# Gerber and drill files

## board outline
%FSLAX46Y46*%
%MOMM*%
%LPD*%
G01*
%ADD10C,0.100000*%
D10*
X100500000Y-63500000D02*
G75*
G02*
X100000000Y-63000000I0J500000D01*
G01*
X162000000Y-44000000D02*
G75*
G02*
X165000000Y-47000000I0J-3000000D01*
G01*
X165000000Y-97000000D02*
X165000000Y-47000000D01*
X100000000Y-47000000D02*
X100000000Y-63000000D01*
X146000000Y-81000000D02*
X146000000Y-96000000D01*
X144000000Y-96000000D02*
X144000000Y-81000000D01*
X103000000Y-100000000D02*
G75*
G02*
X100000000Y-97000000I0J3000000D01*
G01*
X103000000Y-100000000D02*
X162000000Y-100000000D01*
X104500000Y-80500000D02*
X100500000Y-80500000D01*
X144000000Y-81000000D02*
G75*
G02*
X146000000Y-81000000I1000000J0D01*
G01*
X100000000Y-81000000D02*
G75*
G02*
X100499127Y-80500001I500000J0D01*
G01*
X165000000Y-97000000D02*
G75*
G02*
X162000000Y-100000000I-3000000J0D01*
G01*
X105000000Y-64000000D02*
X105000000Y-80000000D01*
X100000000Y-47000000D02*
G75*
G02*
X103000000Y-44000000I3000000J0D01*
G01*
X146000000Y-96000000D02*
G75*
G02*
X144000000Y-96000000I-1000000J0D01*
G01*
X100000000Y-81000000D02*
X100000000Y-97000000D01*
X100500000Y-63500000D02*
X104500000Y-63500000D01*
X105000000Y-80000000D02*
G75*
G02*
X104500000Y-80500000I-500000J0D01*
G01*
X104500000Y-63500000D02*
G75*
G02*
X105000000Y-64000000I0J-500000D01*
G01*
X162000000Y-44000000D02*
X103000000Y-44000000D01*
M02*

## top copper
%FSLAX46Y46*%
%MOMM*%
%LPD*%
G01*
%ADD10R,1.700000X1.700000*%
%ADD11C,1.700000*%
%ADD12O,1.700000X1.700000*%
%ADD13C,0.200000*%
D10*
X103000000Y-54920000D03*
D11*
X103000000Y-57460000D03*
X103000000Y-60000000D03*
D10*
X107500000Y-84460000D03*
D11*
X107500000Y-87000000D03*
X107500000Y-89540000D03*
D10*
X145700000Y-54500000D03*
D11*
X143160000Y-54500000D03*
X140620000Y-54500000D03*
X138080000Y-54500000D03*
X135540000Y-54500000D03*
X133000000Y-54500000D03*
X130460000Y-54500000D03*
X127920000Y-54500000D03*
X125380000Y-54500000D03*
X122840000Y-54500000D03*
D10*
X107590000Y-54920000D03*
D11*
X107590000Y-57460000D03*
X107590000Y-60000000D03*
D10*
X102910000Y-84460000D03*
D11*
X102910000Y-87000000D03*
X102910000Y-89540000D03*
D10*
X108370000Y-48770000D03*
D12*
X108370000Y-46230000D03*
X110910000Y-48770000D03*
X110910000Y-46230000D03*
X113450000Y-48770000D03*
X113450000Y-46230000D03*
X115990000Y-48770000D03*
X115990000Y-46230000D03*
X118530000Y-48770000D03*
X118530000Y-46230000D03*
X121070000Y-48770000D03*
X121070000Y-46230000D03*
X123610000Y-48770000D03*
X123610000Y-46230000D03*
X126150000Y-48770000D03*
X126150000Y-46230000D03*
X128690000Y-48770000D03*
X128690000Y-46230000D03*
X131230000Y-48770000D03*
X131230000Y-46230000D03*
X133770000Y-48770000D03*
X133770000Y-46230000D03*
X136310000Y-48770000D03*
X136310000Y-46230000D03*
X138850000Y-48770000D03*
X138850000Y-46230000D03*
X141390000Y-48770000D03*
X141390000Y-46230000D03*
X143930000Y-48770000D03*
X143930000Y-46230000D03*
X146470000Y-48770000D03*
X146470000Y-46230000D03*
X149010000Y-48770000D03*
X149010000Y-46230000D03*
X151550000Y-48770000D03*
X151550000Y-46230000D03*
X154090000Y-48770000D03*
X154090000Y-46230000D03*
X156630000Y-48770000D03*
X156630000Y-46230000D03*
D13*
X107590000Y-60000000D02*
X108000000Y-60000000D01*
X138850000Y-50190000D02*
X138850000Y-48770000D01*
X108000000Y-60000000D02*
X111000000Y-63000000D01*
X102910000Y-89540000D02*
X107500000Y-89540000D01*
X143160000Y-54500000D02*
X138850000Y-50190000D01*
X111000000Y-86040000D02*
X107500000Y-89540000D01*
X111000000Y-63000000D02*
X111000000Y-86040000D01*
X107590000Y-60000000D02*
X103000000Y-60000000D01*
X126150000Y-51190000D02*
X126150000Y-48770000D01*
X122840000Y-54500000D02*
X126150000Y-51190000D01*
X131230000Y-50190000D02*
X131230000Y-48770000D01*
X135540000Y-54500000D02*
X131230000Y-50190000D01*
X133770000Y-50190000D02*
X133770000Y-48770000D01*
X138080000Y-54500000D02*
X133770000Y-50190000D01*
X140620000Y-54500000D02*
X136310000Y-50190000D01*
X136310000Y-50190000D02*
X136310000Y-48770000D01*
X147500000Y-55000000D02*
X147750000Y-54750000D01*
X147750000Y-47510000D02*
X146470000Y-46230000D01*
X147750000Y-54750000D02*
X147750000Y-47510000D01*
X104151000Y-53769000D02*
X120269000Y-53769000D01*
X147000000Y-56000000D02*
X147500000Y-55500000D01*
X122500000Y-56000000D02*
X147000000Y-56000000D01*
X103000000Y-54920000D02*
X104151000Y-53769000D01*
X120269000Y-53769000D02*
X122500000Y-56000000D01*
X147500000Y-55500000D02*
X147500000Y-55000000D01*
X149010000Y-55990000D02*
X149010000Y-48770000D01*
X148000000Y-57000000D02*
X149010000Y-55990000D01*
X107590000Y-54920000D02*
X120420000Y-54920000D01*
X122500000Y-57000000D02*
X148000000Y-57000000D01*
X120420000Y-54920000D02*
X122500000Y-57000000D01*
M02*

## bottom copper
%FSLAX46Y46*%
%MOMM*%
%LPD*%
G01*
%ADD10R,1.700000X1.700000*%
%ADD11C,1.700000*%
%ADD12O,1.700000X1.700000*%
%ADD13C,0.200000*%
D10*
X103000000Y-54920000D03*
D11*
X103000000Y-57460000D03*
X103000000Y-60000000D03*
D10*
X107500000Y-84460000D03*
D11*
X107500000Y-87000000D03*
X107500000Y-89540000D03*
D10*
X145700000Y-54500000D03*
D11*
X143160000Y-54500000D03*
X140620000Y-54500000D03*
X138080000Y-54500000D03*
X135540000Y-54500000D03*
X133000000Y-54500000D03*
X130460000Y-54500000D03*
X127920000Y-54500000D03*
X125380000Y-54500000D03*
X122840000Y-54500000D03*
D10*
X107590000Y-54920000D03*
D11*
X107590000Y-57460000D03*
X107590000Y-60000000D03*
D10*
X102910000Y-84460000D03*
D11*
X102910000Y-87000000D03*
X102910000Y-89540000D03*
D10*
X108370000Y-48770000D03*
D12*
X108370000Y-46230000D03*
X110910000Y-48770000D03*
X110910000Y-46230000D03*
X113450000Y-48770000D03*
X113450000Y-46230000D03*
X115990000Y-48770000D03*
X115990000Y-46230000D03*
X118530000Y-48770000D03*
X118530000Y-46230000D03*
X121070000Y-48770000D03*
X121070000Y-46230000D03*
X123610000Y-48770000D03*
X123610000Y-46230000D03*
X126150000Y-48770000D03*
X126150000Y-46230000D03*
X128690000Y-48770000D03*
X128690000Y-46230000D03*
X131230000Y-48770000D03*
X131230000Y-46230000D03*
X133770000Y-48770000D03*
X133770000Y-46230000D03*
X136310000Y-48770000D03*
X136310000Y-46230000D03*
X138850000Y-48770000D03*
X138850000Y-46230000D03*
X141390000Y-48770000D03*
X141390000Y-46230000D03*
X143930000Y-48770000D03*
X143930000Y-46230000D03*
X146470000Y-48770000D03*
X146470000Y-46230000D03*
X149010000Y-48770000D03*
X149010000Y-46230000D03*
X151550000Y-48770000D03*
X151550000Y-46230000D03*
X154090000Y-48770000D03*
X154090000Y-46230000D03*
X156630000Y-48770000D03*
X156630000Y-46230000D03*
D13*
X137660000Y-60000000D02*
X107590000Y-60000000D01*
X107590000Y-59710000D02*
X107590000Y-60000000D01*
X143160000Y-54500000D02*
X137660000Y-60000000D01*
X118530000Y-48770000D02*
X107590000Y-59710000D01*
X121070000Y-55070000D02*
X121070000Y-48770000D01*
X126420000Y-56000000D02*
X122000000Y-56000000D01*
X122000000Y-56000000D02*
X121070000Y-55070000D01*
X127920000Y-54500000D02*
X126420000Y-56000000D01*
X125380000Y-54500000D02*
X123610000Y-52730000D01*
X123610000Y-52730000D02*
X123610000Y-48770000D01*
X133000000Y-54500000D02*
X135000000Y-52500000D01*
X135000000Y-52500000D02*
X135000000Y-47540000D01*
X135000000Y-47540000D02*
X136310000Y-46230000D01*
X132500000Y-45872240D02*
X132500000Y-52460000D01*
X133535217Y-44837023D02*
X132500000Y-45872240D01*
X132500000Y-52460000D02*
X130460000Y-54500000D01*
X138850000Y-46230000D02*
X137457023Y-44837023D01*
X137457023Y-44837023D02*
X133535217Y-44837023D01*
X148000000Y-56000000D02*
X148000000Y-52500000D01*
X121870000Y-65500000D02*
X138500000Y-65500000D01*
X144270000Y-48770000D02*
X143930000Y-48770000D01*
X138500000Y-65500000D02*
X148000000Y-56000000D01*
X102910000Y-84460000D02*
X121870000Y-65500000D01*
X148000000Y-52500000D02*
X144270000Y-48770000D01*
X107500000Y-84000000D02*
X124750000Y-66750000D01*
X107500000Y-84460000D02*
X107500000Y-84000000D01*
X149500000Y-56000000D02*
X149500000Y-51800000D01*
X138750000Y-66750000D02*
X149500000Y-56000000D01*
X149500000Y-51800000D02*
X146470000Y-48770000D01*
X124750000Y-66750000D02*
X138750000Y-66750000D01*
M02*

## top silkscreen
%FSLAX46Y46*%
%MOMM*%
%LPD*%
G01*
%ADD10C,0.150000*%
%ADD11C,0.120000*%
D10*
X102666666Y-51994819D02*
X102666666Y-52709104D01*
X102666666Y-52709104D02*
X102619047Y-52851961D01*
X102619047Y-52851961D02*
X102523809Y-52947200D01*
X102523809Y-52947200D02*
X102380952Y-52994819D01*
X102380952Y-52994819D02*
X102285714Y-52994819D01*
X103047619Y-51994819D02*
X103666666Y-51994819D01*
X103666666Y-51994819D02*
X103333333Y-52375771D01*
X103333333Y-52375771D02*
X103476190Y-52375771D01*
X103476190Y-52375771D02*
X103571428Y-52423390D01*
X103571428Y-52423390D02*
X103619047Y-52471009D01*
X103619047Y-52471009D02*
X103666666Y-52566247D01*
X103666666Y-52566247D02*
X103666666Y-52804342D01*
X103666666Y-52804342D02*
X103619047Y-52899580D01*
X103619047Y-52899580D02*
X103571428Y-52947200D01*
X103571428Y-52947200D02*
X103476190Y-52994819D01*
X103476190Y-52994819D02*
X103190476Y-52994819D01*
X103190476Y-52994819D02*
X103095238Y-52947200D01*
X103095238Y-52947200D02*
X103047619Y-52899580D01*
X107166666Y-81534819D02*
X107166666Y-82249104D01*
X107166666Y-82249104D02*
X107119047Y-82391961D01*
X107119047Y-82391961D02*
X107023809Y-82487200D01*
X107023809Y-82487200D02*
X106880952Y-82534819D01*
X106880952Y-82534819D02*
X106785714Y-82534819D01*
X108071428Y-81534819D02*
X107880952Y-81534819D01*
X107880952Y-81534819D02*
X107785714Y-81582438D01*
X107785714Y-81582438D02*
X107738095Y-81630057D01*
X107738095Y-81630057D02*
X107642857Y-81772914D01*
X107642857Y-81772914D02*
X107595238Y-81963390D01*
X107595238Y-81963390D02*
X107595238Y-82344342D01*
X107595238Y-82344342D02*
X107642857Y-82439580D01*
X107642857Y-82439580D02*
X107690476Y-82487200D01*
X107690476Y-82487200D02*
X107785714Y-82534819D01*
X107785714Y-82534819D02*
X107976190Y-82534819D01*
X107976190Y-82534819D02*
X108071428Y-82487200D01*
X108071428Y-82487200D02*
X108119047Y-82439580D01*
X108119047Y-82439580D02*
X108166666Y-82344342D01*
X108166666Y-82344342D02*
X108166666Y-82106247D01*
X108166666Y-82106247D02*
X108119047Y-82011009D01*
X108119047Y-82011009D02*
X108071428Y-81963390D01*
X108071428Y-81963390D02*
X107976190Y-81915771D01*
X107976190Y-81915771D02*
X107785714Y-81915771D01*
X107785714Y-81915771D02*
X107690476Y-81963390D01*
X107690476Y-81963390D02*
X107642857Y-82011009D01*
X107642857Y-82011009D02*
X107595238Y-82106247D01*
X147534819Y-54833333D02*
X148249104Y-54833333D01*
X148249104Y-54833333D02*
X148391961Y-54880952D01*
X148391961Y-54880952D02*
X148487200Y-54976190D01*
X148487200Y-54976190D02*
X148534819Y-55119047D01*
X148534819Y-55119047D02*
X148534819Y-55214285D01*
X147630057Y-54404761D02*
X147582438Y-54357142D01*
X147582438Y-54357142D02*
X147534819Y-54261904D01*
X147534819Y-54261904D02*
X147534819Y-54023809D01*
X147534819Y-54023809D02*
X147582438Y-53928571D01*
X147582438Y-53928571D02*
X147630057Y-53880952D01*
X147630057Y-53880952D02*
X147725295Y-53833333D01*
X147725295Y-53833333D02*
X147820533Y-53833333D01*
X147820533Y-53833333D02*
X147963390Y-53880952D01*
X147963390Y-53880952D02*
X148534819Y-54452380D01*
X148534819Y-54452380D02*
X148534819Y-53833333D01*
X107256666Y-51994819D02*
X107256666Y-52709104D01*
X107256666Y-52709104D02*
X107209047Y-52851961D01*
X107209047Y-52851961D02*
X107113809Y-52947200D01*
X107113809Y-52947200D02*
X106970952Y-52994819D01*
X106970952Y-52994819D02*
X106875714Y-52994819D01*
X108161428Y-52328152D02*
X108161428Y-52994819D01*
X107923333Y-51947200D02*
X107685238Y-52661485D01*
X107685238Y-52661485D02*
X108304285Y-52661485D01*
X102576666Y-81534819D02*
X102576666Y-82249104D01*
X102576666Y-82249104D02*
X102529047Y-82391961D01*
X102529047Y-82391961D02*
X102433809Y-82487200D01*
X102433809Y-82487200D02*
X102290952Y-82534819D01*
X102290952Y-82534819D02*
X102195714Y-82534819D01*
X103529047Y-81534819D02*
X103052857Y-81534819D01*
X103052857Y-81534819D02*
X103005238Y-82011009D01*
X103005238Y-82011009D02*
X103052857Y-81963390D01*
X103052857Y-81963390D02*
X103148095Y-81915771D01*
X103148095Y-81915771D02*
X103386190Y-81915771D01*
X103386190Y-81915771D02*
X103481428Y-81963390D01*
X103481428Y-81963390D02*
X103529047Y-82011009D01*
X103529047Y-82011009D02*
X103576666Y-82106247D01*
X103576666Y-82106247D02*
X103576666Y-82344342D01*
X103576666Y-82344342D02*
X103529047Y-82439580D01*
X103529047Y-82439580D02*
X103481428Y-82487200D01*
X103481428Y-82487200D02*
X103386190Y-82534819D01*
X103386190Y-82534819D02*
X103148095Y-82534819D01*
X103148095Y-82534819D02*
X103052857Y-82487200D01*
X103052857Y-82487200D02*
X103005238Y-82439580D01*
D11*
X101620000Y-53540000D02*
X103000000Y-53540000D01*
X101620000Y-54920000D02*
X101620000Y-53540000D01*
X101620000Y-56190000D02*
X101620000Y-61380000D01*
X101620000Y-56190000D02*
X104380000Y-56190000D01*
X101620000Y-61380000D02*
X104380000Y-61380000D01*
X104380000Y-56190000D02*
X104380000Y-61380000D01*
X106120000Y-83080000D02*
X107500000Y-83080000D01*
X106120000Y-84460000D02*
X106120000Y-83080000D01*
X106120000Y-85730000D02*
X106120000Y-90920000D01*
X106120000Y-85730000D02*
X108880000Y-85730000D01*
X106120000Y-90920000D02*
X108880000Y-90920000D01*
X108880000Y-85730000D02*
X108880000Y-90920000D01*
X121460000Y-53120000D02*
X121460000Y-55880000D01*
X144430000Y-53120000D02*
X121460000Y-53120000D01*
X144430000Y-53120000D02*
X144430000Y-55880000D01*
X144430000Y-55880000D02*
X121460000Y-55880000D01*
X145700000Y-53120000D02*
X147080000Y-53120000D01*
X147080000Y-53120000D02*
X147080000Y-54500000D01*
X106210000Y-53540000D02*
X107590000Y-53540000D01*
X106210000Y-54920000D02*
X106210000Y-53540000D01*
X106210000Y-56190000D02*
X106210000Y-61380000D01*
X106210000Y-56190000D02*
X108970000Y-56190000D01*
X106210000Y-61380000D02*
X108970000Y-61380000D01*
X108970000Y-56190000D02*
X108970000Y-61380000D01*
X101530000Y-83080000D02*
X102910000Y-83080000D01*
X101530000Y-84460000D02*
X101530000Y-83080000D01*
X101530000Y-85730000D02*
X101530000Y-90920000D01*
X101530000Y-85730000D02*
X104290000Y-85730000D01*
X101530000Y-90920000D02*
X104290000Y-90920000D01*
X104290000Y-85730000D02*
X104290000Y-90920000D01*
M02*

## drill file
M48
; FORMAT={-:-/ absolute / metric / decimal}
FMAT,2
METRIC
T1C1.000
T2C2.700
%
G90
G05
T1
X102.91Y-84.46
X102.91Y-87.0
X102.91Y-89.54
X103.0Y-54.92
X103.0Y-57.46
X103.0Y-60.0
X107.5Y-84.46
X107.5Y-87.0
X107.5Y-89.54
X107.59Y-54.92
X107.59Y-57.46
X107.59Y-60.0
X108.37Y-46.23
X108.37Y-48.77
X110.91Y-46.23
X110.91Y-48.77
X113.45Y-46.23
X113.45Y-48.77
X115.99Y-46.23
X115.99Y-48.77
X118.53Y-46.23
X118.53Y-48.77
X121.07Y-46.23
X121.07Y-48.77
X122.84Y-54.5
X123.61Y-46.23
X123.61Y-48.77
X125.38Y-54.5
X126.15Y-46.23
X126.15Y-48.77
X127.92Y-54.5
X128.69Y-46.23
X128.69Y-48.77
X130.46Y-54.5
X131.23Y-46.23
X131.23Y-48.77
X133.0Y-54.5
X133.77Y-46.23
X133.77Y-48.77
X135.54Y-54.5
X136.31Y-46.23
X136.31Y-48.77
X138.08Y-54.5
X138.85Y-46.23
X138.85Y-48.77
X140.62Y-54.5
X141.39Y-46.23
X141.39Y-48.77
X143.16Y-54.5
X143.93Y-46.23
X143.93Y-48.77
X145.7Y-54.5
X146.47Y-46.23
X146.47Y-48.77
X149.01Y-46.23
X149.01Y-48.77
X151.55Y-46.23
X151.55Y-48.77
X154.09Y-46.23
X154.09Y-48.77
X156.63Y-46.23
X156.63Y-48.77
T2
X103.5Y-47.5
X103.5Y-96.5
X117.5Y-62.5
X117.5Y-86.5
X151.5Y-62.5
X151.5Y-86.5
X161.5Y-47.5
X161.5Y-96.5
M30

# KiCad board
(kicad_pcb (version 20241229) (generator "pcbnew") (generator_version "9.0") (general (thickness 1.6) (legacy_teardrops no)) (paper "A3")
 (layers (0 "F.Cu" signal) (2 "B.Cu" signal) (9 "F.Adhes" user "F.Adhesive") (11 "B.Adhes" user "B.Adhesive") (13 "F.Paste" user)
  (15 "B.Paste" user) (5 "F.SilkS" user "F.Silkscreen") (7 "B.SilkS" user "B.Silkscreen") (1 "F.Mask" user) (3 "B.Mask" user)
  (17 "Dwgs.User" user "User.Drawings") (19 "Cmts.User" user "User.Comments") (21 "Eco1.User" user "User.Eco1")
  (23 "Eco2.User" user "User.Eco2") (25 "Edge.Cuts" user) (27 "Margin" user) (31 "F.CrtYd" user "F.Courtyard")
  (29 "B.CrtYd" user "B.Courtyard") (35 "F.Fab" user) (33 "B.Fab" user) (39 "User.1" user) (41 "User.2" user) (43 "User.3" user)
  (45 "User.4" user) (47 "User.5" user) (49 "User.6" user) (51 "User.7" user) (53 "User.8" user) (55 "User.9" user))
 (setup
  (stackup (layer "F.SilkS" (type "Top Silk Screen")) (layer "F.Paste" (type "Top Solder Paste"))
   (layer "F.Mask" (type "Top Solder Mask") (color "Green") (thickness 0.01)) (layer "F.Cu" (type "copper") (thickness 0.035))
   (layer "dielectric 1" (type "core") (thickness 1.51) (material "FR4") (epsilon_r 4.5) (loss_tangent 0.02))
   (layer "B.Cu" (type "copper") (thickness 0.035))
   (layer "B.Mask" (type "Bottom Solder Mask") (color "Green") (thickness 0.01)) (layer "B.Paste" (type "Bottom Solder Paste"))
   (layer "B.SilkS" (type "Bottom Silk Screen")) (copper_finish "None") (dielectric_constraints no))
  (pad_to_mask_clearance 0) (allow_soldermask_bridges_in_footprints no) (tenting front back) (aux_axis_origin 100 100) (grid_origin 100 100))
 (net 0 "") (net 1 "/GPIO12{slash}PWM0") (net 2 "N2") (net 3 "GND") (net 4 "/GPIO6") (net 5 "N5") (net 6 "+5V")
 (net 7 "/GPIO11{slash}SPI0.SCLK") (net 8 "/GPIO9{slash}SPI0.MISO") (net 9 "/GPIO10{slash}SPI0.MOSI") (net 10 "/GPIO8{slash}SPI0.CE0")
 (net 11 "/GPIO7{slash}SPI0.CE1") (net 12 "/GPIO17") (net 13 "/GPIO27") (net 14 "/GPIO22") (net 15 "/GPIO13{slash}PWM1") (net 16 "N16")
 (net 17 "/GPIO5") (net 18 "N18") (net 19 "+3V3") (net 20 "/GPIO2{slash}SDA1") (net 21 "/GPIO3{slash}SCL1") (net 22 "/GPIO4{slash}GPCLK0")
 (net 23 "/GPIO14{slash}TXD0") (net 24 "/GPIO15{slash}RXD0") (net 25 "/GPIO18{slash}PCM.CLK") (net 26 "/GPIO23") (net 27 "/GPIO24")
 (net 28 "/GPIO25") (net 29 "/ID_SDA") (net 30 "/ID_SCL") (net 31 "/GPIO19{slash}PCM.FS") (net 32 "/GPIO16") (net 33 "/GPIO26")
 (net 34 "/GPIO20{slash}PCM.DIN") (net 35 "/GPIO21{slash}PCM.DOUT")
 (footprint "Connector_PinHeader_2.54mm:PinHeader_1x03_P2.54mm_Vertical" (layer "F.Cu") (at 103 54.92)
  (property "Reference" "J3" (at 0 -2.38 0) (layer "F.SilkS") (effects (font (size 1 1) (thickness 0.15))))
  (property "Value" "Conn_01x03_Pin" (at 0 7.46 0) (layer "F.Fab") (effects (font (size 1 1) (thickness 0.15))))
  (fp_line (start -1.38 -1.38) (end 0 -1.38) (stroke (width 0.12) (type solid)) (layer "F.SilkS"))
  (fp_line (start -1.38 0) (end -1.38 -1.38) (stroke (width 0.12) (type solid)) (layer "F.SilkS"))
  (fp_line (start -1.38 1.27) (end -1.38 6.46) (stroke (width 0.12) (type solid)) (layer "F.SilkS"))
  (fp_line (start -1.38 1.27) (end 1.38 1.27) (stroke (width 0.12) (type solid)) (layer "F.SilkS"))
  (fp_line (start -1.38 6.46) (end 1.38 6.46) (stroke (width 0.12) (type solid)) (layer "F.SilkS"))
  (fp_line (start 1.38 1.27) (end 1.38 6.46) (stroke (width 0.12) (type solid)) (layer "F.SilkS"))
  (pad "1" thru_hole rect (at 0 0) (size 1.7 1.7) (drill 1) (layers "*.Cu" "*.Mask") (remove_unused_layers no) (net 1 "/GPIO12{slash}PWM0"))
  (pad "2" thru_hole circle (at 0 2.54) (size 1.7 1.7) (drill 1) (layers "*.Cu" "*.Mask") (remove_unused_layers no) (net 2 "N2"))
  (pad "3" thru_hole circle (at 0 5.08) (size 1.7 1.7) (drill 1) (layers "*.Cu" "*.Mask") (remove_unused_layers no) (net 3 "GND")))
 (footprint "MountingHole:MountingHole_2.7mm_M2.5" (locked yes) (layer "F.Cu") (at 161.5 47.5)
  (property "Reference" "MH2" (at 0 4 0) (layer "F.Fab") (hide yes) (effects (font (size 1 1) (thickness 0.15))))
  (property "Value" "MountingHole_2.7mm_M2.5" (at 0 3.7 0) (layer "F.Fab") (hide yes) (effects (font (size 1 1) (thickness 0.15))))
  (pad "" np_thru_hole circle (at 0 0) (size 2.7 2.7) (drill 2.7) (layers "*.Cu" "*.Mask")))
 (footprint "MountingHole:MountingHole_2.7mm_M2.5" (layer "F.Cu") (at 117.5 86.5)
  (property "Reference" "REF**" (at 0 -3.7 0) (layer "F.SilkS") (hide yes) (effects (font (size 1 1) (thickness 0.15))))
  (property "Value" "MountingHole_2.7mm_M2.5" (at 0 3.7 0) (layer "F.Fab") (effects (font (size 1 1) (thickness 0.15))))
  (pad "" np_thru_hole circle (at 0 0) (size 2.7 2.7) (drill 2.7) (layers "*.Cu" "*.Mask")))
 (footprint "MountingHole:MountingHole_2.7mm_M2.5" (layer "F.Cu") (at 151.5 86.5)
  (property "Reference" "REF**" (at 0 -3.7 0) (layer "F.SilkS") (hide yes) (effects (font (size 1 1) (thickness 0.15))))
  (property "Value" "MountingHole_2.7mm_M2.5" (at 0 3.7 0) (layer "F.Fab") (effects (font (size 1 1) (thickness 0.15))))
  (pad "" np_thru_hole circle (at 0 0) (size 2.7 2.7) (drill 2.7) (layers "*.Cu" "*.Mask")))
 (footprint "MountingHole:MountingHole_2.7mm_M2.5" (layer "F.Cu") (at 151.5 62.5)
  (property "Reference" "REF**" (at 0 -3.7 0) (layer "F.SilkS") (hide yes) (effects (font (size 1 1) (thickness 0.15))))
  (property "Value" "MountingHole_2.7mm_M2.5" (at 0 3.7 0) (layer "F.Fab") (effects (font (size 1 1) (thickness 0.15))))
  (pad "" np_thru_hole circle (at 0 0) (size 2.7 2.7) (drill 2.7) (layers "*.Cu" "*.Mask")))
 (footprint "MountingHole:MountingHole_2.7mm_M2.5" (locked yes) (layer "F.Cu") (at 103.5 96.5)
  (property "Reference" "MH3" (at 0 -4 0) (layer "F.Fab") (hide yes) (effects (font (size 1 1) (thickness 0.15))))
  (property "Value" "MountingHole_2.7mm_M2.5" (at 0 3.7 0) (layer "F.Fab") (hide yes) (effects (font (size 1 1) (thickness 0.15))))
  (pad "" np_thru_hole circle (at 0 0) (size 2.7 2.7) (drill 2.7) (layers "*.Cu" "*.Mask")))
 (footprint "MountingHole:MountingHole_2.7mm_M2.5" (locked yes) (layer "F.Cu") (at 103.5 47.5)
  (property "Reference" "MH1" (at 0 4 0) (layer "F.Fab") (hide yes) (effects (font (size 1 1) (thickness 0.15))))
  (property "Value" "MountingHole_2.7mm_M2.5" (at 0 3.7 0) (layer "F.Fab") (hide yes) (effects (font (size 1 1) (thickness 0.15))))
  (pad "" np_thru_hole circle (at 0 0) (size 2.7 2.7) (drill 2.7) (layers "*.Cu" "*.Mask")))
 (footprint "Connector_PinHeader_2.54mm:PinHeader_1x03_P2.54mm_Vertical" (layer "F.Cu") (at 107.5 84.46)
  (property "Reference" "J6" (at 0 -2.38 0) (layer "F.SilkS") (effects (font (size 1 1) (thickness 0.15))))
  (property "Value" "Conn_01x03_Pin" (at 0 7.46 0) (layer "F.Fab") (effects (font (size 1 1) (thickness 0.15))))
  (fp_line (start -1.38 -1.38) (end 0 -1.38) (stroke (width 0.12) (type solid)) (layer "F.SilkS"))
  (fp_line (start -1.38 0) (end -1.38 -1.38) (stroke (width 0.12) (type solid)) (layer "F.SilkS"))
  (fp_line (start -1.38 1.27) (end -1.38 6.46) (stroke (width 0.12) (type solid)) (layer "F.SilkS"))
  (fp_line (start -1.38 1.27) (end 1.38 1.27) (stroke (width 0.12) (type solid)) (layer "F.SilkS"))
  (fp_line (start -1.38 6.46) (end 1.38 6.46) (stroke (width 0.12) (type solid)) (layer "F.SilkS"))
  (fp_line (start 1.38 1.27) (end 1.38 6.46) (stroke (width 0.12) (type solid)) (layer "F.SilkS"))
  (pad "1" thru_hole rect (at 0 0) (size 1.7 1.7) (drill 1) (layers "*.Cu" "*.Mask") (remove_unused_layers no) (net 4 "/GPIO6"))
  (pad "2" thru_hole circle (at 0 2.54) (size 1.7 1.7) (drill 1) (layers "*.Cu" "*.Mask") (remove_unused_layers no) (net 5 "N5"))
  (pad "3" thru_hole circle (at 0 5.08) (size 1.7 1.7) (drill 1) (layers "*.Cu" "*.Mask") (remove_unused_layers no) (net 3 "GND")))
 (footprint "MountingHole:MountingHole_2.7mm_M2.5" (layer "F.Cu") (at 117.5 62.5)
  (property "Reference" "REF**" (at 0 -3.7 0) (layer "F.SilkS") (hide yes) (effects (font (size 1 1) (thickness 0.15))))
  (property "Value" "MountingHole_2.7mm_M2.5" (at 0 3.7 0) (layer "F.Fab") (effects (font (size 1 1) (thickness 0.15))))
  (pad "" np_thru_hole circle (at 0 0) (size 2.7 2.7) (drill 2.7) (layers "*.Cu" "*.Mask")))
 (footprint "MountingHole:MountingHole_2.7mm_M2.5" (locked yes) (layer "F.Cu") (at 161.5 96.5)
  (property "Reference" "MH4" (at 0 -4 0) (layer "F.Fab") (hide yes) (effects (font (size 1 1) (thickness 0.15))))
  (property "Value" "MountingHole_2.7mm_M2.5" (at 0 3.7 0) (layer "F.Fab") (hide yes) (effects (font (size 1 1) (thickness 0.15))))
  (pad "" np_thru_hole circle (at 0 0) (size 2.7 2.7) (drill 2.7) (layers "*.Cu" "*.Mask")))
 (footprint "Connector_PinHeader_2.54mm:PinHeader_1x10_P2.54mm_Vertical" (layer "F.Cu") (at 145.7 54.5 -90)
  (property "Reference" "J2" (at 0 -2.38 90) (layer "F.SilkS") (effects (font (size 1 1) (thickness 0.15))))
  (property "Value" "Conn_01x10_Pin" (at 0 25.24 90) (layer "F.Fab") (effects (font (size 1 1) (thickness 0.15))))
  (fp_line (start -1.38 24.24) (end 1.38 24.24) (stroke (width 0.12) (type solid)) (layer "F.SilkS"))
  (fp_line (start -1.38 1.27) (end -1.38 24.24) (stroke (width 0.12) (type solid)) (layer "F.SilkS"))
  (fp_line (start -1.38 1.27) (end 1.38 1.27) (stroke (width 0.12) (type solid)) (layer "F.SilkS"))
  (fp_line (start 1.38 1.27) (end 1.38 24.24) (stroke (width 0.12) (type solid)) (layer "F.SilkS"))
  (fp_line (start -1.38 0) (end -1.38 -1.38) (stroke (width 0.12) (type solid)) (layer "F.SilkS"))
  (fp_line (start -1.38 -1.38) (end 0 -1.38) (stroke (width 0.12) (type solid)) (layer "F.SilkS"))
  (pad "1" thru_hole rect (at 0 0 270) (size 1.7 1.7) (drill 1) (layers "*.Cu" "*.Mask") (remove_unused_layers no) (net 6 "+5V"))
  (pad "2" thru_hole circle (at 0 2.54 270) (size 1.7 1.7) (drill 1) (layers "*.Cu" "*.Mask") (remove_unused_layers no) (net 3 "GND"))
  (pad "3" thru_hole circle (at 0 5.08 270) (size 1.7 1.7) (drill 1) (layers "*.Cu" "*.Mask") (remove_unused_layers no)
   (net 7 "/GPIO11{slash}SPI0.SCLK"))
  (pad "4" thru_hole circle (at 0 7.62 270) (size 1.7 1.7) (drill 1) (layers "*.Cu" "*.Mask") (remove_unused_layers no)
   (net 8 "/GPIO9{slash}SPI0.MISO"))
  (pad "5" thru_hole circle (at 0 10.16 270) (size 1.7 1.7) (drill 1) (layers "*.Cu" "*.Mask") (remove_unused_layers no)
   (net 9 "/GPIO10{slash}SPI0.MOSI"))
  (pad "6" thru_hole circle (at 0 12.7 270) (size 1.7 1.7) (drill 1) (layers "*.Cu" "*.Mask") (remove_unused_layers no)
   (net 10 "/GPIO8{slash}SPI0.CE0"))
  (pad "7" thru_hole circle (at 0 15.24 270) (size 1.7 1.7) (drill 1) (layers "*.Cu" "*.Mask") (remove_unused_layers no)
   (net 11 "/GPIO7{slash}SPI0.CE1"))
  (pad "8" thru_hole circle (at 0 17.78 270) (size 1.7 1.7) (drill 1) (layers "*.Cu" "*.Mask") (remove_unused_layers no) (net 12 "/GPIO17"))
  (pad "9" thru_hole circle (at 0 20.32 270) (size 1.7 1.7) (drill 1) (layers "*.Cu" "*.Mask") (remove_unused_layers no) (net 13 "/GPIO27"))
  (pad "10" thru_hole circle (at 0 22.86 270) (size 1.7 1.7) (drill 1) (layers "*.Cu" "*.Mask") (remove_unused_layers no) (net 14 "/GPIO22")))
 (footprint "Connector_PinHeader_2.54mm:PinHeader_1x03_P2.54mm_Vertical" (layer "F.Cu") (at 107.59 54.92)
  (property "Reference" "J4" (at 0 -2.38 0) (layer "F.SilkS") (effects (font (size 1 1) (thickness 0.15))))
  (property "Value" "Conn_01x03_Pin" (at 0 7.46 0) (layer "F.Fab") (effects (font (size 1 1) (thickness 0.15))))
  (fp_line (start -1.38 -1.38) (end 0 -1.38) (stroke (width 0.12) (type solid)) (layer "F.SilkS"))
  (fp_line (start -1.38 0) (end -1.38 -1.38) (stroke (width 0.12) (type solid)) (layer "F.SilkS"))
  (fp_line (start -1.38 1.27) (end -1.38 6.46) (stroke (width 0.12) (type solid)) (layer "F.SilkS"))
  (fp_line (start -1.38 1.27) (end 1.38 1.27) (stroke (width 0.12) (type solid)) (layer "F.SilkS"))
  (fp_line (start -1.38 6.46) (end 1.38 6.46) (stroke (width 0.12) (type solid)) (layer "F.SilkS"))
  (fp_line (start 1.38 1.27) (end 1.38 6.46) (stroke (width 0.12) (type solid)) (layer "F.SilkS"))
  (pad "1" thru_hole rect (at 0 0) (size 1.7 1.7) (drill 1) (layers "*.Cu" "*.Mask") (remove_unused_layers no) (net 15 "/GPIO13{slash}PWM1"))
  (pad "2" thru_hole circle (at 0 2.54) (size 1.7 1.7) (drill 1) (layers "*.Cu" "*.Mask") (remove_unused_layers no) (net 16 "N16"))
  (pad "3" thru_hole circle (at 0 5.08) (size 1.7 1.7) (drill 1) (layers "*.Cu" "*.Mask") (remove_unused_layers no) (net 3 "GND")))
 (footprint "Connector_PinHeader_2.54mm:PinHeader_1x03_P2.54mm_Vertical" (layer "F.Cu") (at 102.91 84.46)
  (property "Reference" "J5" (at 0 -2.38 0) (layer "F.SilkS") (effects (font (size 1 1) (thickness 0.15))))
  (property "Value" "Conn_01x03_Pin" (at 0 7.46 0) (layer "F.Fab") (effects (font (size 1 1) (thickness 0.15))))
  (fp_line (start -1.38 -1.38) (end 0 -1.38) (stroke (width 0.12) (type solid)) (layer "F.SilkS"))
  (fp_line (start -1.38 0) (end -1.38 -1.38) (stroke (width 0.12) (type solid)) (layer "F.SilkS"))
  (fp_line (start -1.38 1.27) (end -1.38 6.46) (stroke (width 0.12) (type solid)) (layer "F.SilkS"))
  (fp_line (start -1.38 1.27) (end 1.38 1.27) (stroke (width 0.12) (type solid)) (layer "F.SilkS"))
  (fp_line (start -1.38 6.46) (end 1.38 6.46) (stroke (width 0.12) (type solid)) (layer "F.SilkS"))
  (fp_line (start 1.38 1.27) (end 1.38 6.46) (stroke (width 0.12) (type solid)) (layer "F.SilkS"))
  (pad "1" thru_hole rect (at 0 0) (size 1.7 1.7) (drill 1) (layers "*.Cu" "*.Mask") (remove_unused_layers no) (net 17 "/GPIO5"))
  (pad "2" thru_hole circle (at 0 2.54) (size 1.7 1.7) (drill 1) (layers "*.Cu" "*.Mask") (remove_unused_layers no) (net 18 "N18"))
  (pad "3" thru_hole circle (at 0 5.08) (size 1.7 1.7) (drill 1) (layers "*.Cu" "*.Mask") (remove_unused_layers no) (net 3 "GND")))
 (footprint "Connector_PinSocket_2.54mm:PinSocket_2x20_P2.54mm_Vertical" (layer "B.Cu") (at 108.37 48.77 -90)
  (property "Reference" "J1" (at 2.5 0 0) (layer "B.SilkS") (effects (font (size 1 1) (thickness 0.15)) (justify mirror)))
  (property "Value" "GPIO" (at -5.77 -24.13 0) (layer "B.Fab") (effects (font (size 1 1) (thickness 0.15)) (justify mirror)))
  (pad "1" thru_hole rect (at 0 0 270) (size 1.7 1.7) (drill 1) (layers "*.Cu" "*.Mask") (remove_unused_layers no) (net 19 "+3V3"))
  (pad "2" thru_hole oval (at -2.54 0 270) (size 1.7 1.7) (drill 1) (layers "*.Cu" "*.Mask") (remove_unused_layers no) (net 6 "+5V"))
  (pad "3" thru_hole oval (at 0 -2.54 270) (size 1.7 1.7) (drill 1) (layers "*.Cu" "*.Mask") (remove_unused_layers no)
   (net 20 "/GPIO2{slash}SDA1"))
  (pad "4" thru_hole oval (at -2.54 -2.54 270) (size 1.7 1.7) (drill 1) (layers "*.Cu" "*.Mask") (remove_unused_layers no) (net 6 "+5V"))
  (pad "5" thru_hole oval (at 0 -5.08 270) (size 1.7 1.7) (drill 1) (layers "*.Cu" "*.Mask") (remove_unused_layers no)
   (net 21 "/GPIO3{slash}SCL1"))
  (pad "6" thru_hole oval (at -2.54 -5.08 270) (size 1.7 1.7) (drill 1) (layers "*.Cu" "*.Mask") (remove_unused_layers no) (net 3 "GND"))
  (pad "7" thru_hole oval (at 0 -7.62 270) (size 1.7 1.7) (drill 1) (layers "*.Cu" "*.Mask") (remove_unused_layers no)
   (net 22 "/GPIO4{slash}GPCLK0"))
  (pad "8" thru_hole oval (at -2.54 -7.62 270) (size 1.7 1.7) (drill 1) (layers "*.Cu" "*.Mask") (remove_unused_layers no)
   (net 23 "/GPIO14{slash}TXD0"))
  (pad "9" thru_hole oval (at 0 -10.16 270) (size 1.7 1.7) (drill 1) (layers "*.Cu" "*.Mask") (remove_unused_layers no) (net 3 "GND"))
  (pad "10" thru_hole oval (at -2.54 -10.16 270) (size 1.7 1.7) (drill 1) (layers "*.Cu" "*.Mask") (remove_unused_layers no)
   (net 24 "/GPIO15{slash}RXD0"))
  (pad "11" thru_hole oval (at 0 -12.7 270) (size 1.7 1.7) (drill 1) (layers "*.Cu" "*.Mask") (remove_unused_layers no) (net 12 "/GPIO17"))
  (pad "12" thru_hole oval (at -2.54 -12.7 270) (size 1.7 1.7) (drill 1) (layers "*.Cu" "*.Mask") (remove_unused_layers no)
   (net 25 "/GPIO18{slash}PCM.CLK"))
  (pad "13" thru_hole oval (at 0 -15.24 270) (size 1.7 1.7) (drill 1) (layers "*.Cu" "*.Mask") (remove_unused_layers no) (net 13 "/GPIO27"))
  (pad "14" thru_hole oval (at -2.54 -15.24 270) (size 1.7 1.7) (drill 1) (layers "*.Cu" "*.Mask") (remove_unused_layers no) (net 3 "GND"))
  (pad "15" thru_hole oval (at 0 -17.78 270) (size 1.7 1.7) (drill 1) (layers "*.Cu" "*.Mask") (remove_unused_layers no) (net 14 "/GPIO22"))
  (pad "16" thru_hole oval (at -2.54 -17.78 270) (size 1.7 1.7) (drill 1) (layers "*.Cu" "*.Mask") (remove_unused_layers no)
   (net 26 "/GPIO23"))
  (pad "17" thru_hole oval (at 0 -20.32 270) (size 1.7 1.7) (drill 1) (layers "*.Cu" "*.Mask") (remove_unused_layers no) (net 19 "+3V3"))
  (pad "18" thru_hole oval (at -2.54 -20.32 270) (size 1.7 1.7) (drill 1) (layers "*.Cu" "*.Mask") (remove_unused_layers no)
   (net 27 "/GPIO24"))
  (pad "19" thru_hole oval (at 0 -22.86 270) (size 1.7 1.7) (drill 1) (layers "*.Cu" "*.Mask") (remove_unused_layers no)
   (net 9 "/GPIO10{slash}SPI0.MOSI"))
  (pad "20" thru_hole oval (at -2.54 -22.86 270) (size 1.7 1.7) (drill 1) (layers "*.Cu" "*.Mask") (remove_unused_layers no) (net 3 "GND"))
  (pad "21" thru_hole oval (at 0 -25.4 270) (size 1.7 1.7) (drill 1) (layers "*.Cu" "*.Mask") (remove_unused_layers no)
   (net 8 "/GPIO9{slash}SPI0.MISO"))
  (pad "22" thru_hole oval (at -2.54 -25.4 270) (size 1.7 1.7) (drill 1) (layers "*.Cu" "*.Mask") (remove_unused_layers no)
   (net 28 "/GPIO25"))
  (pad "23" thru_hole oval (at 0 -27.94 270) (size 1.7 1.7) (drill 1) (layers "*.Cu" "*.Mask") (remove_unused_layers no)
   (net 7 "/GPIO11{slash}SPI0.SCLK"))
  (pad "24" thru_hole oval (at -2.54 -27.94 270) (size 1.7 1.7) (drill 1) (layers "*.Cu" "*.Mask") (remove_unused_layers no)
   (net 10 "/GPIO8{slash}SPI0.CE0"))
  (pad "25" thru_hole oval (at 0 -30.48 270) (size 1.7 1.7) (drill 1) (layers "*.Cu" "*.Mask") (remove_unused_layers no) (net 3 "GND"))
  (pad "26" thru_hole oval (at -2.54 -30.48 270) (size 1.7 1.7) (drill 1) (layers "*.Cu" "*.Mask") (remove_unused_layers no)
   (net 11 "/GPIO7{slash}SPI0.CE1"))
  (pad "27" thru_hole oval (at 0 -33.02 270) (size 1.7 1.7) (drill 1) (layers "*.Cu" "*.Mask") (remove_unused_layers no) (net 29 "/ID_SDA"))
  (pad "28" thru_hole oval (at -2.54 -33.02 270) (size 1.7 1.7) (drill 1) (layers "*.Cu" "*.Mask") (remove_unused_layers no)
   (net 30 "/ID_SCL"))
  (pad "29" thru_hole oval (at 0 -35.56 270) (size 1.7 1.7) (drill 1) (layers "*.Cu" "*.Mask") (remove_unused_layers no) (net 17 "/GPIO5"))
  (pad "30" thru_hole oval (at -2.54 -35.56 270) (size 1.7 1.7) (drill 1) (layers "*.Cu" "*.Mask") (remove_unused_layers no) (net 3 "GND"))
  (pad "31" thru_hole oval (at 0 -38.1 270) (size 1.7 1.7) (drill 1) (layers "*.Cu" "*.Mask") (remove_unused_layers no) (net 4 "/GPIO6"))
  (pad "32" thru_hole oval (at -2.54 -38.1 270) (size 1.7 1.7) (drill 1) (layers "*.Cu" "*.Mask") (remove_unused_layers no)
   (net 1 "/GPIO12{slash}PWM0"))
  (pad "33" thru_hole oval (at 0 -40.64 270) (size 1.7 1.7) (drill 1) (layers "*.Cu" "*.Mask") (remove_unused_layers no)
   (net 15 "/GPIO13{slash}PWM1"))
  (pad "34" thru_hole oval (at -2.54 -40.64 270) (size 1.7 1.7) (drill 1) (layers "*.Cu" "*.Mask") (remove_unused_layers no) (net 3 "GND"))
  (pad "35" thru_hole oval (at 0 -43.18 270) (size 1.7 1.7) (drill 1) (layers "*.Cu" "*.Mask") (remove_unused_layers no)
   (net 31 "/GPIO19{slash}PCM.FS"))
  (pad "36" thru_hole oval (at -2.54 -43.18 270) (size 1.7 1.7) (drill 1) (layers "*.Cu" "*.Mask") (remove_unused_layers no)
   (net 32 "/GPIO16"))
  (pad "37" thru_hole oval (at 0 -45.72 270) (size 1.7 1.7) (drill 1) (layers "*.Cu" "*.Mask") (remove_unused_layers no) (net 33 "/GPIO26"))
  (pad "38" thru_hole oval (at -2.54 -45.72 270) (size 1.7 1.7) (drill 1) (layers "*.Cu" "*.Mask") (remove_unused_layers no)
   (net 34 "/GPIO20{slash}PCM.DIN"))
  (pad "39" thru_hole oval (at 0 -48.26 270) (size 1.7 1.7) (drill 1) (layers "*.Cu" "*.Mask") (remove_unused_layers no) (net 3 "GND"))
  (pad "40" thru_hole oval (at -2.54 -48.26 270) (size 1.7 1.7) (drill 1) (layers "*.Cu" "*.Mask") (remove_unused_layers no)
   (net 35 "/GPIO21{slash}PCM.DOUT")))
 (gr_arc (start 100.5 63.5) (mid 100.146447 63.353553) (end 100 63) (stroke (width 0.1) (type solid)) (layer "Edge.Cuts"))
 (gr_arc (start 162 44) (mid 164.12132 44.87868) (end 165 47) (stroke (width 0.1) (type solid)) (layer "Edge.Cuts"))
 (gr_line (start 165 97) (end 165 47) (stroke (width 0.1) (type solid)) (layer "Edge.Cuts"))
 (gr_line (start 100 47) (end 100 63) (stroke (width 0.1) (type solid)) (layer "Edge.Cuts"))
 (gr_line (start 146 81) (end 146 96) (stroke (width 0.1) (type solid)) (layer "Edge.Cuts"))
 (gr_line (start 144 96) (end 144 81) (stroke (width 0.1) (type solid)) (layer "Edge.Cuts"))
 (gr_arc (start 103 100) (mid 100.87868 99.12132) (end 100 97) (stroke (width 0.1) (type solid)) (layer "Edge.Cuts"))
 (gr_line (start 103 100) (end 162 100) (stroke (width 0.1) (type solid)) (layer "Edge.Cuts"))
 (gr_line (start 104.5 80.5) (end 100.5 80.5) (stroke (width 0.1) (type solid)) (layer "Edge.Cuts"))
 (gr_arc (start 144 81) (mid 145 80) (end 146 81) (stroke (width 0.1) (type solid)) (layer "Edge.Cuts"))
 (gr_arc (start 100 81) (mid 100.146138 80.646755) (end 100.499127 80.500001) (stroke (width 0.1) (type solid)) (layer "Edge.Cuts"))
 (gr_arc (start 165 97) (mid 164.12132 99.12132) (end 162 100) (stroke (width 0.1) (type solid)) (layer "Edge.Cuts"))
 (gr_line (start 105 64) (end 105 80) (stroke (width 0.1) (type solid)) (layer "Edge.Cuts"))
 (gr_arc (start 100 47) (mid 100.87868 44.87868) (end 103 44) (stroke (width 0.1) (type solid)) (layer "Edge.Cuts"))
 (gr_arc (start 146 96) (mid 145 97) (end 144 96) (stroke (width 0.1) (type solid)) (layer "Edge.Cuts"))
 (gr_line (start 100 81) (end 100 97) (stroke (width 0.1) (type solid)) (layer "Edge.Cuts"))
 (gr_line (start 100.5 63.5) (end 104.5 63.5) (stroke (width 0.1) (type solid)) (layer "Edge.Cuts"))
 (gr_arc (start 105 80) (mid 104.853553 80.353553) (end 104.5 80.5) (stroke (width 0.1) (type solid)) (layer "Edge.Cuts"))
 (gr_arc (start 104.5 63.5) (mid 104.853553 63.646447) (end 105 64) (stroke (width 0.1) (type solid)) (layer "Edge.Cuts"))
 (gr_line (start 162 44) (end 103 44) (stroke (width 0.1) (type solid)) (layer "Edge.Cuts"))
 (segment (start 107.59 60) (end 108 60) (width 0.2) (layer "F.Cu") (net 3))
 (segment (start 138.85 50.19) (end 138.85 48.77) (width 0.2) (layer "F.Cu") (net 3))
 (segment (start 108 60) (end 111 63) (width 0.2) (layer "F.Cu") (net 3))
 (segment (start 102.91 89.54) (end 107.5 89.54) (width 0.2) (layer "F.Cu") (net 3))
 (segment (start 143.16 54.5) (end 138.85 50.19) (width 0.2) (layer "F.Cu") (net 3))
 (segment (start 111 86.04) (end 107.5 89.54) (width 0.2) (layer "F.Cu") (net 3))
 (segment (start 111 63) (end 111 86.04) (width 0.2) (layer "F.Cu") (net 3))
 (segment (start 107.59 60) (end 103 60) (width 0.2) (layer "F.Cu") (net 3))
 (segment (start 137.66 60) (end 107.59 60) (width 0.2) (layer "B.Cu") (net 3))
 (segment (start 107.59 59.71) (end 107.59 60) (width 0.2) (layer "B.Cu") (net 3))
 (segment (start 143.16 54.5) (end 137.66 60) (width 0.2) (layer "B.Cu") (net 3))
 (segment (start 118.53 48.77) (end 107.59 59.71) (width 0.2) (layer "B.Cu") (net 3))
 (segment (start 121.07 55.07) (end 121.07 48.77) (width 0.2) (layer "B.Cu") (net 12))
 (segment (start 126.42 56) (end 122 56) (width 0.2) (layer "B.Cu") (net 12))
 (segment (start 122 56) (end 121.07 55.07) (width 0.2) (layer "B.Cu") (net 12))
 (segment (start 127.92 54.5) (end 126.42 56) (width 0.2) (layer "B.Cu") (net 12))
 (segment (start 125.38 54.5) (end 123.61 52.73) (width 0.2) (layer "B.Cu") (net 13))
 (segment (start 123.61 52.73) (end 123.61 48.77) (width 0.2) (layer "B.Cu") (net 13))
 (segment (start 126.15 51.19) (end 126.15 48.77) (width 0.2) (layer "F.Cu") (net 14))
 (segment (start 122.84 54.5) (end 126.15 51.19) (width 0.2) (layer "F.Cu") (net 14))
 (segment (start 131.23 50.19) (end 131.23 48.77) (width 0.2) (layer "F.Cu") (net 9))
 (segment (start 135.54 54.5) (end 131.23 50.19) (width 0.2) (layer "F.Cu") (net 9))
 (segment (start 133.77 50.19) (end 133.77 48.77) (width 0.2) (layer "F.Cu") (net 8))
 (segment (start 138.08 54.5) (end 133.77 50.19) (width 0.2) (layer "F.Cu") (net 8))
 (segment (start 140.62 54.5) (end 136.31 50.19) (width 0.2) (layer "F.Cu") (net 7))
 (segment (start 136.31 50.19) (end 136.31 48.77) (width 0.2) (layer "F.Cu") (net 7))
 (segment (start 133 54.5) (end 135 52.5) (width 0.2) (layer "B.Cu") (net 10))
 (segment (start 135 52.5) (end 135 47.54) (width 0.2) (layer "B.Cu") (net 10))
 (segment (start 135 47.54) (end 136.31 46.23) (width 0.2) (layer "B.Cu") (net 10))
 (segment (start 132.5 45.87224) (end 132.5 52.46) (width 0.2) (layer "B.Cu") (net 11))
 (segment (start 133.535217 44.837023) (end 132.5 45.87224) (width 0.2) (layer "B.Cu") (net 11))
 (segment (start 132.5 52.46) (end 130.46 54.5) (width 0.2) (layer "B.Cu") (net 11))
 (segment (start 138.85 46.23) (end 137.457023 44.837023) (width 0.2) (layer "B.Cu") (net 11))
 (segment (start 137.457023 44.837023) (end 133.535217 44.837023) (width 0.2) (layer "B.Cu") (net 11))
 (segment (start 148 56) (end 148 52.5) (width 0.2) (layer "B.Cu") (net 17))
 (segment (start 121.87 65.5) (end 138.5 65.5) (width 0.2) (layer "B.Cu") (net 17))
 (segment (start 144.27 48.77) (end 143.93 48.77) (width 0.2) (layer "B.Cu") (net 17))
 (segment (start 138.5 65.5) (end 148 56) (width 0.2) (layer "B.Cu") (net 17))
 (segment (start 102.91 84.46) (end 121.87 65.5) (width 0.2) (layer "B.Cu") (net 17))
 (segment (start 148 52.5) (end 144.27 48.77) (width 0.2) (layer "B.Cu") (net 17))
 (segment (start 107.5 84) (end 124.75 66.75) (width 0.2) (layer "B.Cu") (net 4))
 (segment (start 107.5 84.46) (end 107.5 84) (width 0.2) (layer "B.Cu") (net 4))
 (segment (start 149.5 56) (end 149.5 51.8) (width 0.2) (layer "B.Cu") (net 4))
 (segment (start 138.75 66.75) (end 149.5 56) (width 0.2) (layer "B.Cu") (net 4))
 (segment (start 149.5 51.8) (end 146.47 48.77) (width 0.2) (layer "B.Cu") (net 4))
 (segment (start 124.75 66.75) (end 138.75 66.75) (width 0.2) (layer "B.Cu") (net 4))
 (segment (start 147.5 55) (end 147.75 54.75) (width 0.2) (layer "F.Cu") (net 1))
 (segment (start 147.75 47.51) (end 146.47 46.23) (width 0.2) (layer "F.Cu") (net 1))
 (segment (start 147.75 54.75) (end 147.75 47.51) (width 0.2) (layer "F.Cu") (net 1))
 (segment (start 104.151 53.769) (end 120.269 53.769) (width 0.2) (layer "F.Cu") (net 1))
 (segment (start 147 56) (end 147.5 55.5) (width 0.2) (layer "F.Cu") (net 1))
 (segment (start 122.5 56) (end 147 56) (width 0.2) (layer "F.Cu") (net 1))
 (segment (start 103 54.92) (end 104.151 53.769) (width 0.2) (layer "F.Cu") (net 1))
 (segment (start 120.269 53.769) (end 122.5 56) (width 0.2) (layer "F.Cu") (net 1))
 (segment (start 147.5 55.5) (end 147.5 55) (width 0.2) (layer "F.Cu") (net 1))
 (segment (start 149.01 55.99) (end 149.01 48.77) (width 0.2) (layer "F.Cu") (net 15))
 (segment (start 148 57) (end 149.01 55.99) (width 0.2) (layer "F.Cu") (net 15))
 (segment (start 107.59 54.92) (end 120.42 54.92) (width 0.2) (layer "F.Cu") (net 15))
 (segment (start 122.5 57) (end 148 57) (width 0.2) (layer "F.Cu") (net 15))
 (segment (start 120.42 54.92) (end 122.5 57) (width 0.2) (layer "F.Cu") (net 15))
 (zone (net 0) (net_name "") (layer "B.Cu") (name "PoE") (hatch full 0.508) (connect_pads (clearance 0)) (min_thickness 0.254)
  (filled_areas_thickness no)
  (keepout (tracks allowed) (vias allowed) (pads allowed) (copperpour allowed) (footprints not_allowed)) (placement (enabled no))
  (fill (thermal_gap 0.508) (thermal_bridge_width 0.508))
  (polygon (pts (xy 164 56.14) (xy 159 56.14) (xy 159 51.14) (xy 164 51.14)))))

